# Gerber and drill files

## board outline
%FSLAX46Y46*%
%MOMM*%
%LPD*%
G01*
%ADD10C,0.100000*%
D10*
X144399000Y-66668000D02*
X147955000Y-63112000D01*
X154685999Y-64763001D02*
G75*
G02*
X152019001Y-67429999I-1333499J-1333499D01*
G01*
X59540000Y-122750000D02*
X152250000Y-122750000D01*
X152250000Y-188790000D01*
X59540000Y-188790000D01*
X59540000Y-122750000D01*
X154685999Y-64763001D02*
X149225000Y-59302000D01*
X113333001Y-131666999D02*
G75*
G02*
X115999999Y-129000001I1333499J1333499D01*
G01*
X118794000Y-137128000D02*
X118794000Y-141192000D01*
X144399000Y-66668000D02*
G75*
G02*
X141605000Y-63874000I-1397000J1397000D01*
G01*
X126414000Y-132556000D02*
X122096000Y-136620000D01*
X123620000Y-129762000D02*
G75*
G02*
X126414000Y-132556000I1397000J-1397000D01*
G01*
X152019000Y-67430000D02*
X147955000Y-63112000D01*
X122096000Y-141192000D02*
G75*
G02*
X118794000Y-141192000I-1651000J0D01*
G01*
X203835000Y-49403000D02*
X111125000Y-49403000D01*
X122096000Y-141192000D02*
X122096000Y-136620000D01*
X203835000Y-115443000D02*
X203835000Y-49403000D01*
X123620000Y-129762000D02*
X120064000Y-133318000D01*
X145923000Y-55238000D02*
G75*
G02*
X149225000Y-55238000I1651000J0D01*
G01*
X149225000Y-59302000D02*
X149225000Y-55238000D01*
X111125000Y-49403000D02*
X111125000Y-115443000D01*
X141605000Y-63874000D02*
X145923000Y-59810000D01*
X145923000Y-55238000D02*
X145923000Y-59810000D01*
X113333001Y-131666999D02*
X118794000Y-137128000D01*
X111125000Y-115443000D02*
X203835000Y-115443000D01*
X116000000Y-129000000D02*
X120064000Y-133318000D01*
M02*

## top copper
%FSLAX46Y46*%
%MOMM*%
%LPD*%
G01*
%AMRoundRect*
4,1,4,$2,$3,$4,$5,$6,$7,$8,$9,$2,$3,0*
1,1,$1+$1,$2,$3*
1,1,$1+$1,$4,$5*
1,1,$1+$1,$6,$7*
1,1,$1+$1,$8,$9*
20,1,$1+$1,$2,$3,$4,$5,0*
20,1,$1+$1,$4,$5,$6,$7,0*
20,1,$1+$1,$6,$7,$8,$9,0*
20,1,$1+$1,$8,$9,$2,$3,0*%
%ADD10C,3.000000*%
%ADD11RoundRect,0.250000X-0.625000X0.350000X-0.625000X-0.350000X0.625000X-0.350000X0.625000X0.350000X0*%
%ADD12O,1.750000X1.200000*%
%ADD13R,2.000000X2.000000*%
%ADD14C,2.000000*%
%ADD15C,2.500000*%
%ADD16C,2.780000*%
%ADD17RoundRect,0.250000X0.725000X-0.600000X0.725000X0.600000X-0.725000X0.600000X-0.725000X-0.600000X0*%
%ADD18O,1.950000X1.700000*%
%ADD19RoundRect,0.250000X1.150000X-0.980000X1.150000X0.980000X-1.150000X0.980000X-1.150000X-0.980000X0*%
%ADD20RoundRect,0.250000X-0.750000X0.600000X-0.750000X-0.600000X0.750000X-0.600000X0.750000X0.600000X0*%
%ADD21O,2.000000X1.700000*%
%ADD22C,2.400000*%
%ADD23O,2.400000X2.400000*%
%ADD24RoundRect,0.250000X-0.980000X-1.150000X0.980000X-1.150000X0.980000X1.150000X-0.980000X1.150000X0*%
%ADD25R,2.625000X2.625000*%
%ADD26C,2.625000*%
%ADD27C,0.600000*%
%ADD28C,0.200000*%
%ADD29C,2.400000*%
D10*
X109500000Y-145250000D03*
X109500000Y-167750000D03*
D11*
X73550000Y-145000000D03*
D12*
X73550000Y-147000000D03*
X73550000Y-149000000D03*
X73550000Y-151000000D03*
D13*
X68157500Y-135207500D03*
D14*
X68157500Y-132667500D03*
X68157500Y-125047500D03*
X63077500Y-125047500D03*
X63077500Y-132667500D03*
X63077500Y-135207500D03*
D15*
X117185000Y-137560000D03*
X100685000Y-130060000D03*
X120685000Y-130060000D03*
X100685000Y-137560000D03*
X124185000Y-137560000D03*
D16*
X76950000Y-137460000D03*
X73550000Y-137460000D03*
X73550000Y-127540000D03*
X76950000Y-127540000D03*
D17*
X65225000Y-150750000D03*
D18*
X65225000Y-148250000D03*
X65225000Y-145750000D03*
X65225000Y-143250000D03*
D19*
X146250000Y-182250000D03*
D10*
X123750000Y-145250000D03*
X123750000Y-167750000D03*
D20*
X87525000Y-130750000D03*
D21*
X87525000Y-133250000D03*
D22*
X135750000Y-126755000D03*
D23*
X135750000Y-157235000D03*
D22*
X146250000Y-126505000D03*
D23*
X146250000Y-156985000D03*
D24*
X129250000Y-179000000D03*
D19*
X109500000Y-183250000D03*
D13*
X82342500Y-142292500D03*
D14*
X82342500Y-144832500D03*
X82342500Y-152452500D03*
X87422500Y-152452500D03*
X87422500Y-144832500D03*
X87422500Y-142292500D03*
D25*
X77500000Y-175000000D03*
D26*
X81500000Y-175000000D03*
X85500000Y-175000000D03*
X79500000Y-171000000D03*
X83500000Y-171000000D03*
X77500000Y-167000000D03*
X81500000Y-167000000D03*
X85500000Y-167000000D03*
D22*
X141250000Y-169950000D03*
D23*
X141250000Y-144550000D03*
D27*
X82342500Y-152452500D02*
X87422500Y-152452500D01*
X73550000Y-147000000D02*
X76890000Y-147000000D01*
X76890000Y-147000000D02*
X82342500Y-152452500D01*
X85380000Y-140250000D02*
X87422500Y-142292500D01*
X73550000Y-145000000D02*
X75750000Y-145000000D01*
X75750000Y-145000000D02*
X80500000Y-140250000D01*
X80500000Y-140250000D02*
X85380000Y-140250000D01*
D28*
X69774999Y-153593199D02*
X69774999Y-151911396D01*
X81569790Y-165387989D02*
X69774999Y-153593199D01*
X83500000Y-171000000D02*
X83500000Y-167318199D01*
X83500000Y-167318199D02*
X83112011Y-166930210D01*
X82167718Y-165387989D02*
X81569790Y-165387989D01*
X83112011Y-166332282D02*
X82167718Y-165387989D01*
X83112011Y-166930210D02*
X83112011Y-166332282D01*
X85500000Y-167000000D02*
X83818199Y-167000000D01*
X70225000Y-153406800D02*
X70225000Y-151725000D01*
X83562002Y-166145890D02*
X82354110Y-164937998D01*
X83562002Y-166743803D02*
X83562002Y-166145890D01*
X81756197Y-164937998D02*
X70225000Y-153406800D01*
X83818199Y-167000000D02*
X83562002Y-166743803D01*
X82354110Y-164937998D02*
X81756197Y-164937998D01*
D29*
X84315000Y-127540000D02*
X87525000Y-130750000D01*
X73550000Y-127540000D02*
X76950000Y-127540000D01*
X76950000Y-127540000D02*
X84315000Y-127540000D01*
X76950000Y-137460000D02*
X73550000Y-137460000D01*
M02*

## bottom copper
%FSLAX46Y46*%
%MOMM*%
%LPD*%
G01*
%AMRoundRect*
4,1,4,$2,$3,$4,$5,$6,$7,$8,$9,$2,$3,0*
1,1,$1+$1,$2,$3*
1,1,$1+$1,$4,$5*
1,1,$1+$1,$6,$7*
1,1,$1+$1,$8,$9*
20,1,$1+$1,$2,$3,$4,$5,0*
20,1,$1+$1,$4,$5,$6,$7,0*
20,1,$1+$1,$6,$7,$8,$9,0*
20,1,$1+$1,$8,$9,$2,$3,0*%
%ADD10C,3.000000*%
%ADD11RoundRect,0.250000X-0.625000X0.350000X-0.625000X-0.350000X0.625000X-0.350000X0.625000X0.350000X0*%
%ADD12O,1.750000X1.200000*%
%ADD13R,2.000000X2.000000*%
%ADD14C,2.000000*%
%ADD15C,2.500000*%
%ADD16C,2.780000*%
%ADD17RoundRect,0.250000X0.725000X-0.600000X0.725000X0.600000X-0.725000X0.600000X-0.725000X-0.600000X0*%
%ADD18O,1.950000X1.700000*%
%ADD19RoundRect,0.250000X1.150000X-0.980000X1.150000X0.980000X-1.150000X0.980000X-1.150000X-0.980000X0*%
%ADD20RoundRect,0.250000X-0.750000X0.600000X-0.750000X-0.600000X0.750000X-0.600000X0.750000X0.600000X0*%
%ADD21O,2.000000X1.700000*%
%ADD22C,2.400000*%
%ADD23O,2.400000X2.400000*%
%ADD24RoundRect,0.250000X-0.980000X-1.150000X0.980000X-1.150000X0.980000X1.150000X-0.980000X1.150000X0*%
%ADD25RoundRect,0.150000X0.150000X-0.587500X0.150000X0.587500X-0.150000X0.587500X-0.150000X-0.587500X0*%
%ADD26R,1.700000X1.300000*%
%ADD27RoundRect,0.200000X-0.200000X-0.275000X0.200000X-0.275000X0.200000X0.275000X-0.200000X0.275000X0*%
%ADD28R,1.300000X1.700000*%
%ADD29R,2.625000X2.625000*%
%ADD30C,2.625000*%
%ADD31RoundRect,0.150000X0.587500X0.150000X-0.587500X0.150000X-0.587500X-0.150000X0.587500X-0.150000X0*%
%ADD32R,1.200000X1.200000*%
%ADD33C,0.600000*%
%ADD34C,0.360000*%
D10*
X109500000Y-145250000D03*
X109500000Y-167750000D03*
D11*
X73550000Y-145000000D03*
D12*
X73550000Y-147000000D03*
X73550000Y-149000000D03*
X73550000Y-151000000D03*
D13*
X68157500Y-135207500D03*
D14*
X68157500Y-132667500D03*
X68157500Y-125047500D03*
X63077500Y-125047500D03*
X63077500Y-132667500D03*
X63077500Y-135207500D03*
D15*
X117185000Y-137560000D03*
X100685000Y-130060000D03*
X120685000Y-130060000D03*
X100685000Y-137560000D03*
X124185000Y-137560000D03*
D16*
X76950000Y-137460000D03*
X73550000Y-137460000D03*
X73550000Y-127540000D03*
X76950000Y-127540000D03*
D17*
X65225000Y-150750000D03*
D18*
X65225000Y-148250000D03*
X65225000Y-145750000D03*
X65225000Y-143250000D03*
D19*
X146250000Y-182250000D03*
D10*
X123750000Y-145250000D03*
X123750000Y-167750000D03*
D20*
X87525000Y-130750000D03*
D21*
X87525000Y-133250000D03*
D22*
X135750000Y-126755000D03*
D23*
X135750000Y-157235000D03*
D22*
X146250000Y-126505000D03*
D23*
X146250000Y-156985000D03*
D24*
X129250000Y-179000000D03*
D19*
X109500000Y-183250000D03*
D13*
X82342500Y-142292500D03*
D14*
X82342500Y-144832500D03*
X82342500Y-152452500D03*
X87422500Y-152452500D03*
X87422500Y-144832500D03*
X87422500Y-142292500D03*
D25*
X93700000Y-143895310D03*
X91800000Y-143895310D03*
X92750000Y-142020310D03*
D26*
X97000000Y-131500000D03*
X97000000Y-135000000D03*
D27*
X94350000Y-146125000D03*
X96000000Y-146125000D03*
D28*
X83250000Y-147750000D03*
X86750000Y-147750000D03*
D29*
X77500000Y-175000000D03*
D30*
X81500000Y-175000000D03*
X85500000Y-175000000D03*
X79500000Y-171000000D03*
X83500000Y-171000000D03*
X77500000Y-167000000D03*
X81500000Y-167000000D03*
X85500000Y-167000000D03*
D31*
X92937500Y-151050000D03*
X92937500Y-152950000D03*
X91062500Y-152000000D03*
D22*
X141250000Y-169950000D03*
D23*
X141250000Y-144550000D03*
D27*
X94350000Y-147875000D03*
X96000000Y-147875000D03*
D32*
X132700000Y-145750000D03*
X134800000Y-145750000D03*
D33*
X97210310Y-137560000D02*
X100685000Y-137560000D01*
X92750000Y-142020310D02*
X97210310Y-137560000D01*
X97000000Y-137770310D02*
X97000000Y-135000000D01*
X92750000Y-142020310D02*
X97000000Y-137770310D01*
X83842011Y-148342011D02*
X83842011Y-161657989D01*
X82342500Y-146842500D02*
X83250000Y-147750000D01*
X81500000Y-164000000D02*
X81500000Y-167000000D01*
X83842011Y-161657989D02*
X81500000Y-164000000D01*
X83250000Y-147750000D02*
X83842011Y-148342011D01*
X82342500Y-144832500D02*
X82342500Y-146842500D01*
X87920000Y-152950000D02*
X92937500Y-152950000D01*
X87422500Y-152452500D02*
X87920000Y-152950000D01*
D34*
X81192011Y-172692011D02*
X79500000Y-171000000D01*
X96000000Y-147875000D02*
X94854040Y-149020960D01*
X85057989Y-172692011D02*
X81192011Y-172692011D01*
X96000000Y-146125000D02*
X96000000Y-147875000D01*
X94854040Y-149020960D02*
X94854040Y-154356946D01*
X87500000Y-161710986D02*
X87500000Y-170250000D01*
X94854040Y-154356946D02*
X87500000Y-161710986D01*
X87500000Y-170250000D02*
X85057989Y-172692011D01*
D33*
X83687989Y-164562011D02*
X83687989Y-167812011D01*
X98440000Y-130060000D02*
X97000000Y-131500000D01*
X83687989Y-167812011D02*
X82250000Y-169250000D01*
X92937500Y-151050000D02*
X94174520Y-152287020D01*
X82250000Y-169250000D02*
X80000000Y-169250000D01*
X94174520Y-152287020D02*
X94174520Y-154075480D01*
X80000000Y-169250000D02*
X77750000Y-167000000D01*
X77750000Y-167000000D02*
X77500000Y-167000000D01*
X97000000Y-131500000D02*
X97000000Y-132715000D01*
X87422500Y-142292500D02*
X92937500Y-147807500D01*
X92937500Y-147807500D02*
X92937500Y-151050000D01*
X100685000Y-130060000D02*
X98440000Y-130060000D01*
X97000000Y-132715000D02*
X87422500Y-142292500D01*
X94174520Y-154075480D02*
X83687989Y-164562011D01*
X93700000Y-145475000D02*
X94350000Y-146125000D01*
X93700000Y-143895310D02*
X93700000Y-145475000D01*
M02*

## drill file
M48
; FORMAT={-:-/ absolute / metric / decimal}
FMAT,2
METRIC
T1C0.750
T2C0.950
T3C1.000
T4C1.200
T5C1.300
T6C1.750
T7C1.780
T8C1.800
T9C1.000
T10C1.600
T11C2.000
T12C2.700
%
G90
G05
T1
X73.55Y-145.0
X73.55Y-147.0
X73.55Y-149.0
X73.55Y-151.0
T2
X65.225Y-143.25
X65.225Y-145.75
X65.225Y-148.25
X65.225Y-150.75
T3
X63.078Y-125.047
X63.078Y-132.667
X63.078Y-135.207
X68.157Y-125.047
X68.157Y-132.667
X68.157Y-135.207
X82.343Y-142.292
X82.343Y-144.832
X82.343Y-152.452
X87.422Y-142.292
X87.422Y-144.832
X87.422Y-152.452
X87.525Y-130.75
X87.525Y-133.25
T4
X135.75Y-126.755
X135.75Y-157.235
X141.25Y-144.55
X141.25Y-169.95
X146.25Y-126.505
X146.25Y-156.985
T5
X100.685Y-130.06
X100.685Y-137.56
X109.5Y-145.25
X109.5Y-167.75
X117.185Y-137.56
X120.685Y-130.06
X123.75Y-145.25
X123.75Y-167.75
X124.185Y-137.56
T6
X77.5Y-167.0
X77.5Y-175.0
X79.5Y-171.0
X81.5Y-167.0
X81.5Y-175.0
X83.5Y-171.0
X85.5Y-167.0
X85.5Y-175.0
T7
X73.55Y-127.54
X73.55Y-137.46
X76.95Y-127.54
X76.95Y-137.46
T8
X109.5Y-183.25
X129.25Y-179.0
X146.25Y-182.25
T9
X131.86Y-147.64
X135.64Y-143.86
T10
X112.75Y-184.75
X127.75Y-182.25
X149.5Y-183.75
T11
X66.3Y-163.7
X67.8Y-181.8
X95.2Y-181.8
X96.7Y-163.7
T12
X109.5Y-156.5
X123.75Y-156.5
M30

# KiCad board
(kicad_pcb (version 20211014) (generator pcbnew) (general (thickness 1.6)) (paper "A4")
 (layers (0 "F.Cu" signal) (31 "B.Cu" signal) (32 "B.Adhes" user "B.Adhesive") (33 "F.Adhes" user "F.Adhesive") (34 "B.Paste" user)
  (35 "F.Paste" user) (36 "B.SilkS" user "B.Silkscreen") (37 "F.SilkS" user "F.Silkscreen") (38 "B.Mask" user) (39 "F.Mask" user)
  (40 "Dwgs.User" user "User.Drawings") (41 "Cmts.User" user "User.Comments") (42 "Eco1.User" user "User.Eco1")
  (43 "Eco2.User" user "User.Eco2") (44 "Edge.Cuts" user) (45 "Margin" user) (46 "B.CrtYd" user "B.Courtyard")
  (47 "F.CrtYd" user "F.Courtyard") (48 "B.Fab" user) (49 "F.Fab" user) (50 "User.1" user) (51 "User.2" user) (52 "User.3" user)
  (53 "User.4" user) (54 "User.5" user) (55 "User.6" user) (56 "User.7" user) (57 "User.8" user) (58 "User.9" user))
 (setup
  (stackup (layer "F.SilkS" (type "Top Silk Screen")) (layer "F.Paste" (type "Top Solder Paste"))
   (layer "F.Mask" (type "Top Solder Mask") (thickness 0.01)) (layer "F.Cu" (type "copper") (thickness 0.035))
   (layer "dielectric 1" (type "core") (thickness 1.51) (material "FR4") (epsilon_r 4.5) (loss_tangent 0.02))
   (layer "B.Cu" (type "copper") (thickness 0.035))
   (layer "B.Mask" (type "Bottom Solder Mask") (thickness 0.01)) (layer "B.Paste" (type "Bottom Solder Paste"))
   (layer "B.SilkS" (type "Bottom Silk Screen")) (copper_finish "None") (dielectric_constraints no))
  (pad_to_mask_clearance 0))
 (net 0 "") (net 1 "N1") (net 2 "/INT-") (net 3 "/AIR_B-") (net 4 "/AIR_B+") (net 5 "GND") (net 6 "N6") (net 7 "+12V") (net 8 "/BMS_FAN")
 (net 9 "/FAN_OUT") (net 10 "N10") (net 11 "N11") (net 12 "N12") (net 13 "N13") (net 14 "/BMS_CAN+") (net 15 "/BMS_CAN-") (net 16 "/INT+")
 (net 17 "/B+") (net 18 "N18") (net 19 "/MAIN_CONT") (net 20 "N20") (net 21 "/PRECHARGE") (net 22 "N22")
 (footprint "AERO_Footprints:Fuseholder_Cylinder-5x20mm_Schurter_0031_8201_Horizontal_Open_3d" (layer "F.Cu") (at 109.5 145.25 -90)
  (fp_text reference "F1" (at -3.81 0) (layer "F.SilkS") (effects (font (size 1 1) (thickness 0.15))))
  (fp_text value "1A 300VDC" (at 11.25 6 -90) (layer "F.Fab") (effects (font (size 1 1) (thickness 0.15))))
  (pad "" np_thru_hole circle locked (at 11.25 0 270) (size 2.7 2.7) (drill 2.7) (layers *.Cu *.Mask))
  (pad "1" thru_hole circle locked (at 0 0 270) (size 3 3) (drill 1.3) (layers *.Cu *.Mask) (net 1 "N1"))
  (pad "2" thru_hole circle locked (at 22.5 0 270) (size 3 3) (drill 1.3) (layers *.Cu *.Mask) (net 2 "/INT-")))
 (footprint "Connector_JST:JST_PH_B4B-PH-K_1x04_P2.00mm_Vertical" (layer "F.Cu") (at 73.55 145 -90)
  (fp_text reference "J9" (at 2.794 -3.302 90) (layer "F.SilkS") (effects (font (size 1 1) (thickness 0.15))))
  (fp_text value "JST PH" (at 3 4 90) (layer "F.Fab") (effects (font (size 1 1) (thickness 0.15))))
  (pad "1" thru_hole roundrect locked (at 0 0 270) (size 1.2 1.75) (drill 0.75) (layers *.Cu *.Mask) (roundrect_rratio 0.208333)
   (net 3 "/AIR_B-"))
  (pad "2" thru_hole oval locked (at 2 0 270) (size 1.2 1.75) (drill 0.75) (layers *.Cu *.Mask) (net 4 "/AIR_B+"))
  (pad "3" thru_hole oval locked (at 4 0 270) (size 1.2 1.75) (drill 0.75) (layers *.Cu *.Mask) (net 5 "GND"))
  (pad "4" thru_hole oval locked (at 6 0 270) (size 1.2 1.75) (drill 0.75) (layers *.Cu *.Mask) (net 5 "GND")))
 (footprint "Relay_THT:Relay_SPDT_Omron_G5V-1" (layer "F.Cu") (at 68.1575 135.2075 180)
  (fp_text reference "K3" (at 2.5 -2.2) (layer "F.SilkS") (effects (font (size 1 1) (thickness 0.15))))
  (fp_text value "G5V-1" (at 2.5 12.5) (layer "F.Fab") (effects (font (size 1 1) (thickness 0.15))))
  (pad "1" thru_hole rect locked (at 0 0 180) (size 2 2) (drill 1) (layers *.Cu *.Mask) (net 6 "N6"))
  (pad "2" thru_hole circle locked (at 0 2.54 180) (size 2 2) (drill 1) (layers *.Cu *.Mask) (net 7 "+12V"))
  (pad "5" thru_hole circle locked (at 0 10.16 180) (size 2 2) (drill 1) (layers *.Cu *.Mask) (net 7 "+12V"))
  (pad "6" thru_hole circle locked (at 5.08 10.16 180) (size 2 2) (drill 1) (layers *.Cu *.Mask) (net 7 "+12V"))
  (pad "9" thru_hole circle locked (at 5.08 2.54 180) (size 2 2) (drill 1) (layers *.Cu *.Mask) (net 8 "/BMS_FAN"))
  (pad "10" thru_hole circle locked (at 5.08 0 180) (size 2 2) (drill 1) (layers *.Cu *.Mask) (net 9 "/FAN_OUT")))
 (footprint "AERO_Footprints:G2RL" (layer "F.Cu") (at 113.385 133.75)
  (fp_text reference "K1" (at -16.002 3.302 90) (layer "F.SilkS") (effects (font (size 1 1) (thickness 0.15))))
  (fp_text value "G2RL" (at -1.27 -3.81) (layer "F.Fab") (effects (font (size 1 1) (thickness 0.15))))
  (pad "1" thru_hole circle locked (at 3.8 3.81) (size 2.5 2.5) (drill 1.3) (layers *.Cu *.Mask) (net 1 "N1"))
  (pad "2" thru_hole circle locked (at -12.7 -3.69) (size 2.5 2.5) (drill 1.3) (layers *.Cu *.Mask) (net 3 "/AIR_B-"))
  (pad "5" thru_hole circle locked (at 7.3 -3.69) (size 2.5 2.5) (drill 1.3) (layers *.Cu *.Mask) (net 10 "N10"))
  (pad "9" thru_hole circle locked (at -12.7 3.81) (size 2.5 2.5) (drill 1.3) (layers *.Cu *.Mask) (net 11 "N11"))
  (pad "10" thru_hole circle locked (at 10.8 3.81) (size 2.5 2.5) (drill 1.3) (layers *.Cu *.Mask) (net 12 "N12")))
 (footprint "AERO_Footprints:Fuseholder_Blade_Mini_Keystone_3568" (layer "F.Cu") (at 73.55 137.46 90)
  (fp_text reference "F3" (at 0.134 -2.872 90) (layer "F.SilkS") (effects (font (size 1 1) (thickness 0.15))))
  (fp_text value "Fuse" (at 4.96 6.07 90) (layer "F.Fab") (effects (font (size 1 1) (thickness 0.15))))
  (pad "1" thru_hole circle locked (at 0 3.4 90) (size 2.78 2.78) (drill 1.78) (layers *.Cu *.Mask) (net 9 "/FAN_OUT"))
  (pad "1" thru_hole circle locked (at 0 0 90) (size 2.78 2.78) (drill 1.78) (layers *.Cu *.Mask) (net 9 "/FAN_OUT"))
  (pad "2" thru_hole circle locked (at 9.92 0 90) (size 2.78 2.78) (drill 1.78) (layers *.Cu *.Mask) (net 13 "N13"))
  (pad "2" thru_hole circle locked (at 9.92 3.4 90) (size 2.78 2.78) (drill 1.78) (layers *.Cu *.Mask) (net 13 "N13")))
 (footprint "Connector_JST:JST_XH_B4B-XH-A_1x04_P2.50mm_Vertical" (layer "F.Cu") (at 65.225 150.75 90)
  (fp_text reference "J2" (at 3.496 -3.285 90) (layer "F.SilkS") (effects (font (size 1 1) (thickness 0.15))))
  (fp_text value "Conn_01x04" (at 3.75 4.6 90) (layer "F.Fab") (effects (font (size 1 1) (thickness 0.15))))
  (pad "1" thru_hole roundrect locked (at 0 0 90) (size 1.7 1.95) (drill 0.95) (layers *.Cu *.Mask) (roundrect_rratio 0.147059)
   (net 7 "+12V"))
  (pad "2" thru_hole oval locked (at 2.5 0 90) (size 1.7 1.95) (drill 0.95) (layers *.Cu *.Mask) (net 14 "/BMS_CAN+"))
  (pad "3" thru_hole oval locked (at 5 0 90) (size 1.7 1.95) (drill 0.95) (layers *.Cu *.Mask) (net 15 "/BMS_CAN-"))
  (pad "4" thru_hole oval locked (at 7.5 0 90) (size 1.7 1.95) (drill 0.95) (layers *.Cu *.Mask) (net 5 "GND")))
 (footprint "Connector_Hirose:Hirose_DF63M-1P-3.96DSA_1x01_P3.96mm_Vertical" (layer "F.Cu") (at 146.25 182.25 90)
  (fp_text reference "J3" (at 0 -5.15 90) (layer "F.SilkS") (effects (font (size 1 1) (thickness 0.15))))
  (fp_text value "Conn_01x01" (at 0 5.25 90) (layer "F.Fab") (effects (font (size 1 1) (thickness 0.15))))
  (pad "" np_thru_hole circle locked (at -1.5 3.25 90) (size 1.6 1.6) (drill 1.6) (layers *.Cu *.Mask))
  (pad "1" thru_hole roundrect locked (at 0 0 90) (size 2.46 2.8) (drill 1.8) (layers *.Cu *.Mask) (roundrect_rratio 0.101626)
   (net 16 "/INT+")))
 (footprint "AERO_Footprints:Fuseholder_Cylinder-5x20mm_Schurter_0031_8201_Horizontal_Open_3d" (layer "F.Cu") (at 123.75 145.25 -90)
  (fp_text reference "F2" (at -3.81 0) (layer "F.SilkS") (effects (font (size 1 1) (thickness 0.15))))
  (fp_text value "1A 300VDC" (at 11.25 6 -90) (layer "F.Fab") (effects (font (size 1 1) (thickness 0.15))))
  (pad "" np_thru_hole circle locked (at 11.25 0 270) (size 2.7 2.7) (drill 2.7) (layers *.Cu *.Mask))
  (pad "1" thru_hole circle locked (at 0 0 270) (size 3 3) (drill 1.3) (layers *.Cu *.Mask) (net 12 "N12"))
  (pad "2" thru_hole circle locked (at 22.5 0 270) (size 3 3) (drill 1.3) (layers *.Cu *.Mask) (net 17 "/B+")))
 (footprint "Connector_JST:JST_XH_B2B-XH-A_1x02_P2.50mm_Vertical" (layer "F.Cu") (at 87.525 130.75 -90)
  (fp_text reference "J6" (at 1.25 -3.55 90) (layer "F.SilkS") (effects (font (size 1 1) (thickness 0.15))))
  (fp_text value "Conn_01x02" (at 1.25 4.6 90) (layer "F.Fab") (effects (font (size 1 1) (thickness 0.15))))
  (pad "1" thru_hole roundrect locked (at 0 0 270) (size 1.7 2) (drill 1) (layers *.Cu *.Mask) (roundrect_rratio 0.147059) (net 13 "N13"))
  (pad "2" thru_hole oval locked (at 2.5 0 270) (size 1.7 2) (drill 1) (layers *.Cu *.Mask) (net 5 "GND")))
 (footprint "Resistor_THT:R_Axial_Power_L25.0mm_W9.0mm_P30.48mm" (layer "F.Cu") (at 135.75 126.755 -90)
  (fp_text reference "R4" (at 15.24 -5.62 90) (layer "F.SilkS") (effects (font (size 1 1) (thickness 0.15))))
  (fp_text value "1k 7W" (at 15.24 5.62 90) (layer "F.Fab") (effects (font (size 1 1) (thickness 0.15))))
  (pad "1" thru_hole circle locked (at 0 0 270) (size 2.4 2.4) (drill 1.2) (layers *.Cu *.Mask) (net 10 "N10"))
  (pad "2" thru_hole oval locked (at 30.48 0 270) (size 2.4 2.4) (drill 1.2) (layers *.Cu *.Mask) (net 16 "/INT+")))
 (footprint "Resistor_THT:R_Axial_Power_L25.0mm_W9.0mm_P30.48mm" (layer "F.Cu") (at 146.25 126.505 -90)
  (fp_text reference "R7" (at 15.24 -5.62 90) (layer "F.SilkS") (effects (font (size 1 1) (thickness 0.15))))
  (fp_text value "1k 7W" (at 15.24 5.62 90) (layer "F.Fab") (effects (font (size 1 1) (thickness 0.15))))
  (pad "1" thru_hole circle locked (at 0 0 270) (size 2.4 2.4) (drill 1.2) (layers *.Cu *.Mask) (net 10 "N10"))
  (pad "2" thru_hole oval locked (at 30.48 0 270) (size 2.4 2.4) (drill 1.2) (layers *.Cu *.Mask) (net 16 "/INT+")))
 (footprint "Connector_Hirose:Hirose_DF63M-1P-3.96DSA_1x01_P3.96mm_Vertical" (layer "F.Cu") (at 129.25 179)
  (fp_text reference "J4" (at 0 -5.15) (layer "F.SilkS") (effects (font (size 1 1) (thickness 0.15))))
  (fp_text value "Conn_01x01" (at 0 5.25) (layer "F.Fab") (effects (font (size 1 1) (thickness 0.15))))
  (pad "" np_thru_hole circle locked (at -1.5 3.25) (size 1.6 1.6) (drill 1.6) (layers *.Cu *.Mask))
  (pad "1" thru_hole roundrect locked (at 0 0) (size 2.46 2.8) (drill 1.8) (layers *.Cu *.Mask) (roundrect_rratio 0.101626) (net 17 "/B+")))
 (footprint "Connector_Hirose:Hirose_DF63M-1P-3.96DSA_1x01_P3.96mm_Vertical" (layer "F.Cu") (at 109.5 183.25 90)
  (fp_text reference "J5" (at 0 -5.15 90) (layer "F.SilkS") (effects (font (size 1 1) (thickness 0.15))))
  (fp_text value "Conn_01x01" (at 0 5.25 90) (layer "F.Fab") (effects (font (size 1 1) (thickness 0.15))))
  (pad "" np_thru_hole circle locked (at -1.5 3.25 90) (size 1.6 1.6) (drill 1.6) (layers *.Cu *.Mask))
  (pad "1" thru_hole roundrect locked (at 0 0 90) (size 2.46 2.8) (drill 1.8) (layers *.Cu *.Mask) (roundrect_rratio 0.101626)
   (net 2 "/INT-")))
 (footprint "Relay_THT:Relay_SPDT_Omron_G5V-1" (layer "F.Cu") (at 82.3425 142.2925)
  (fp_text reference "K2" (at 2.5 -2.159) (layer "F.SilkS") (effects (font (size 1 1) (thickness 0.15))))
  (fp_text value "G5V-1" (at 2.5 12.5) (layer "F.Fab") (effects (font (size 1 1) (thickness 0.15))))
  (pad "1" thru_hole rect locked (at 0 0) (size 2 2) (drill 1) (layers *.Cu *.Mask) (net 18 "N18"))
  (pad "2" thru_hole circle locked (at 0 2.54) (size 2 2) (drill 1) (layers *.Cu *.Mask) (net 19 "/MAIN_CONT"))
  (pad "5" thru_hole circle locked (at 0 10.16) (size 2 2) (drill 1) (layers *.Cu *.Mask) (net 4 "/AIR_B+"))
  (pad "6" thru_hole circle locked (at 5.08 10.16) (size 2 2) (drill 1) (layers *.Cu *.Mask) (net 4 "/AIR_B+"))
  (pad "9" thru_hole circle locked (at 5.08 2.54) (size 2 2) (drill 1) (layers *.Cu *.Mask) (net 5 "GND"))
  (pad "10" thru_hole circle locked (at 5.08 0) (size 2 2) (drill 1) (layers *.Cu *.Mask) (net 3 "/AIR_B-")))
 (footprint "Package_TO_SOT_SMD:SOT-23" (layer "B.Cu") (at 92.75 142.95781 90)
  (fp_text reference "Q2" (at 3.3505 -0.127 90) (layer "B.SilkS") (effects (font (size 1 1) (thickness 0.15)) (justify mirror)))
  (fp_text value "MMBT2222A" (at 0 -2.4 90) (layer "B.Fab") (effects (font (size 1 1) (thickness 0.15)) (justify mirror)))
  (pad "1" smd roundrect locked (at -0.9375 0.95 90) (size 1.475 0.6) (layers "B.Cu" "B.Paste" "B.Mask") (roundrect_rratio 0.25)
   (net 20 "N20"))
  (pad "2" smd roundrect locked (at -0.9375 -0.95 90) (size 1.475 0.6) (layers "B.Cu" "B.Paste" "B.Mask") (roundrect_rratio 0.25)
   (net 5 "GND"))
  (pad "3" smd roundrect locked (at 0.9375 0 90) (size 1.475 0.6) (layers "B.Cu" "B.Paste" "B.Mask") (roundrect_rratio 0.25) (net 11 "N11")))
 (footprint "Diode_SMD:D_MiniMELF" (layer "B.Cu") (at 97 133.25 -90)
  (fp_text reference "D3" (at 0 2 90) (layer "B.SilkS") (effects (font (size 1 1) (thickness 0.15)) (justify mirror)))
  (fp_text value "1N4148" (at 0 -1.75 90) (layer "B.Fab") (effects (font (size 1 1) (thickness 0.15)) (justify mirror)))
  (pad "1" smd rect locked (at -1.75 0 270) (size 1.3 1.7) (layers "B.Cu" "B.Paste" "B.Mask") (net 3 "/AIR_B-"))
  (pad "2" smd rect locked (at 1.75 0 270) (size 1.3 1.7) (layers "B.Cu" "B.Paste" "B.Mask") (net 11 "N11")))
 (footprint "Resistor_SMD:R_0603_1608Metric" (layer "B.Cu") (at 95.175 146.125)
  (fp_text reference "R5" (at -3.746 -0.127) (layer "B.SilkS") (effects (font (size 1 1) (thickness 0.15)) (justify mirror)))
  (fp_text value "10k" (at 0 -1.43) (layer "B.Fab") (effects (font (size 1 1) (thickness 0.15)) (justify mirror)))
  (pad "1" smd roundrect locked (at -0.825 0) (size 0.8 0.95) (layers "B.Cu" "B.Paste" "B.Mask") (roundrect_rratio 0.25) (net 20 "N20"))
  (pad "2" smd roundrect locked (at 0.825 0) (size 0.8 0.95) (layers "B.Cu" "B.Paste" "B.Mask") (roundrect_rratio 0.25)
   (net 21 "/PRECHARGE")))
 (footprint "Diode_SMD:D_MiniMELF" (layer "B.Cu") (at 85 147.75)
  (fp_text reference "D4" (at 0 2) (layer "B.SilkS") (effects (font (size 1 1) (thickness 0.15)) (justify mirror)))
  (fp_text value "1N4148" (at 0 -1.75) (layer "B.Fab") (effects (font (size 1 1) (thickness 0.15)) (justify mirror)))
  (pad "1" smd rect locked (at -1.75 0) (size 1.3 1.7) (layers "B.Cu" "B.Paste" "B.Mask") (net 19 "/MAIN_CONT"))
  (pad "2" smd rect locked (at 1.75 0) (size 1.3 1.7) (layers "B.Cu" "B.Paste" "B.Mask") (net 5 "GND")))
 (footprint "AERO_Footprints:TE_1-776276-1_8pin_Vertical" (layer "B.Cu") (at 81.5 171)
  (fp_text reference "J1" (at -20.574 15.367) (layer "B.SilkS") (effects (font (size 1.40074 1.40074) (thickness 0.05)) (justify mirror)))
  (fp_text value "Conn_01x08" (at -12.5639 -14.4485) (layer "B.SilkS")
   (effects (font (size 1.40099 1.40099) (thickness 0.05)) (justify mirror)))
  (pad "" np_thru_hole circle locked (at 13.7 10.8) (size 2 2) (drill 2) (layers *.Cu *.Mask "B.SilkS"))
  (pad "" np_thru_hole circle locked (at -15.2 -7.3) (size 2 2) (drill 2) (layers *.Cu *.Mask "B.SilkS"))
  (pad "" np_thru_hole circle locked (at 15.2 -7.3) (size 2 2) (drill 2) (layers *.Cu *.Mask "B.SilkS"))
  (pad "" np_thru_hole circle locked (at -13.7 10.8) (size 2 2) (drill 2) (layers *.Cu *.Mask "B.SilkS"))
  (pad "1" thru_hole rect locked (at -4 4) (size 2.625 2.625) (drill 1.75) (layers *.Cu *.Mask) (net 5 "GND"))
  (pad "2" thru_hole circle locked (at 0 4) (size 2.625 2.625) (drill 1.75) (layers *.Cu *.Mask) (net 8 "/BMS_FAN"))
  (pad "3" thru_hole circle locked (at 4 4) (size 2.625 2.625) (drill 1.75) (layers *.Cu *.Mask) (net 7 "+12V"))
  (pad "4" thru_hole circle locked (at -2 0) (size 2.625 2.625) (drill 1.75) (layers *.Cu *.Mask) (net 21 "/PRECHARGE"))
  (pad "5" thru_hole circle locked (at 2 0) (size 2.625 2.625) (drill 1.75) (layers *.Cu *.Mask) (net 14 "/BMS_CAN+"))
  (pad "6" thru_hole circle locked (at -4 -4) (size 2.625 2.625) (drill 1.75) (layers *.Cu *.Mask) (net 3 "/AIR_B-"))
  (pad "7" thru_hole circle locked (at 0 -4) (size 2.625 2.625) (drill 1.75) (layers *.Cu *.Mask) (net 19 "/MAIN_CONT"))
  (pad "8" thru_hole circle locked (at 4 -4) (size 2.625 2.625) (drill 1.75) (layers *.Cu *.Mask) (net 15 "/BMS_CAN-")))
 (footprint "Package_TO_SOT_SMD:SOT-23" (layer "B.Cu") (at 92 152 180)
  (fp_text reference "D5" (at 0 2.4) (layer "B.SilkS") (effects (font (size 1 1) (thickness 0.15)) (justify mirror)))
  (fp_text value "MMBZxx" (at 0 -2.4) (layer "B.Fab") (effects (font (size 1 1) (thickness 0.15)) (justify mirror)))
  (pad "1" smd roundrect locked (at -0.9375 0.95 180) (size 1.475 0.6) (layers "B.Cu" "B.Paste" "B.Mask") (roundrect_rratio 0.25)
   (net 3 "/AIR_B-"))
  (pad "2" smd roundrect locked (at -0.9375 -0.95 180) (size 1.475 0.6) (layers "B.Cu" "B.Paste" "B.Mask") (roundrect_rratio 0.25)
   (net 4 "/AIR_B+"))
  (pad "3" smd roundrect locked (at 0.9375 0 180) (size 1.475 0.6) (layers "B.Cu" "B.Paste" "B.Mask") (roundrect_rratio 0.25) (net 5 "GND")))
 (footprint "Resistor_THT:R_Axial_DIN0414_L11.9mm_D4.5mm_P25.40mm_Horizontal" (layer "B.Cu") (at 141.25 169.95 90)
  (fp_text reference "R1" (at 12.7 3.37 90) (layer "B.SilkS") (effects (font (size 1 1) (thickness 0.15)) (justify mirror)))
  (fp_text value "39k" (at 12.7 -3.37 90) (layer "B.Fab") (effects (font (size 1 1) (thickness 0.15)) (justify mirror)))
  (pad "1" thru_hole circle locked (at 0 0 90) (size 2.4 2.4) (drill 1.2) (layers *.Cu *.Mask) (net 16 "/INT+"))
  (pad "2" thru_hole oval locked (at 25.4 0 90) (size 2.4 2.4) (drill 1.2) (layers *.Cu *.Mask) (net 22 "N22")))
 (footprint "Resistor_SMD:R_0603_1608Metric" (layer "B.Cu") (at 95.175 147.875)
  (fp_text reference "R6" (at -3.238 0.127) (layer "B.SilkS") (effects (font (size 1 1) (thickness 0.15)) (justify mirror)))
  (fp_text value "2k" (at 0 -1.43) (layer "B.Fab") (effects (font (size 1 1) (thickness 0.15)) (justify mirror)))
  (pad "1" smd roundrect locked (at -0.825 0) (size 0.8 0.95) (layers "B.Cu" "B.Paste" "B.Mask") (roundrect_rratio 0.25) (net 5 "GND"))
  (pad "2" smd roundrect locked (at 0.825 0) (size 0.8 0.95) (layers "B.Cu" "B.Paste" "B.Mask") (roundrect_rratio 0.25)
   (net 21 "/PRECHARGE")))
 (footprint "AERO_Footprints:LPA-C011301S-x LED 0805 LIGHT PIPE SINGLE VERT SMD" (layer "B.Cu") (at 133.75 145.75)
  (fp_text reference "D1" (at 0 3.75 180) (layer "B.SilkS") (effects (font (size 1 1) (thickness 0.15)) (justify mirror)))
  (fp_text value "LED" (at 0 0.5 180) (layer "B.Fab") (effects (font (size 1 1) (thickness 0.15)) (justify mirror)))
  (pad "" np_thru_hole circle locked (at 1.89 -1.89) (size 1 1) (drill 1) (layers *.Cu *.Mask))
  (pad "" np_thru_hole circle locked (at -1.89 1.89) (size 1 1) (drill 1) (layers *.Cu *.Mask))
  (pad "1" smd rect locked (at -1.05 0) (size 1.2 1.2) (layers "B.Cu" "B.Paste" "B.Mask") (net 2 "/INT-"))
  (pad "2" smd rect locked (at 1.05 0) (size 1.2 1.2) (layers "B.Cu" "B.Paste" "B.Mask") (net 22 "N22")))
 (gr_line (start 144.399 66.668) (end 147.955 63.112) (layer "Edge.Cuts") (width 0.1))
 (gr_arc (start 154.685999 64.763001) (mid 154.685999 67.429999) (end 152.019001 67.429999) (layer "Edge.Cuts") (width 0.1))
 (gr_rect (start 59.54 188.79) (end 152.25 122.75) (layer "Edge.Cuts") (width 0.1) (fill none))
 (gr_line (start 154.685999 64.763001) (end 149.225 59.302) (layer "Edge.Cuts") (width 0.1))
 (gr_arc (start 113.333001 131.666999) (mid 113.333001 129.000001) (end 115.999999 129.000001) (layer "Edge.Cuts") (width 0.1))
 (gr_line (start 118.794 137.128) (end 118.794 141.192) (layer "Edge.Cuts") (width 0.1))
 (gr_arc (start 144.399 66.668) (mid 141.605 66.668) (end 141.605 63.874) (layer "Edge.Cuts") (width 0.1))
 (gr_line (start 126.414 132.556) (end 122.096 136.62) (layer "Edge.Cuts") (width 0.1))
 (gr_arc (start 123.62 129.762) (mid 126.414 129.762) (end 126.414 132.556) (layer "Edge.Cuts") (width 0.1))
 (gr_line (start 152.019 67.43) (end 147.955 63.112) (layer "Edge.Cuts") (width 0.1))
 (gr_arc (start 122.096 141.192) (mid 120.445 142.843) (end 118.794 141.192) (layer "Edge.Cuts") (width 0.1))
 (gr_line (start 203.835 49.403) (end 111.125 49.403) (layer "Edge.Cuts") (width 0.1))
 (gr_line (start 122.096 141.192) (end 122.096 136.62) (layer "Edge.Cuts") (width 0.1))
 (gr_line (start 203.835 115.443) (end 203.835 49.403) (layer "Edge.Cuts") (width 0.1))
 (gr_line (start 123.62 129.762) (end 120.064 133.318) (layer "Edge.Cuts") (width 0.1))
 (gr_arc (start 145.923 55.238) (mid 147.574 53.587) (end 149.225 55.238) (layer "Edge.Cuts") (width 0.1))
 (gr_line (start 149.225 59.302) (end 149.225 55.238) (layer "Edge.Cuts") (width 0.1))
 (gr_line (start 111.125 49.403) (end 111.125 115.443) (layer "Edge.Cuts") (width 0.1))
 (gr_line (start 141.605 63.874) (end 145.923 59.81) (layer "Edge.Cuts") (width 0.1))
 (gr_line (start 145.923 55.238) (end 145.923 59.81) (layer "Edge.Cuts") (width 0.1))
 (gr_line (start 113.333001 131.666999) (end 118.794 137.128) (layer "Edge.Cuts") (width 0.1))
 (gr_line (start 111.125 115.443) (end 203.835 115.443) (layer "Edge.Cuts") (width 0.1))
 (gr_line (start 116 129) (end 120.064 133.318) (layer "Edge.Cuts") (width 0.1))
 (segment (start 97.21031 137.56) (end 100.685 137.56) (width 0.6) (layer "B.Cu") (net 11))
 (segment (start 92.75 142.02031) (end 97.21031 137.56) (width 0.6) (layer "B.Cu") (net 11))
 (segment (start 97 137.77031) (end 97 135) (width 0.6) (layer "B.Cu") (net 11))
 (segment (start 92.75 142.02031) (end 97 137.77031) (width 0.6) (layer "B.Cu") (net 11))
 (segment (start 83.842011 148.342011) (end 83.842011 161.657989) (width 0.6) (layer "B.Cu") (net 19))
 (segment (start 82.3425 146.8425) (end 83.25 147.75) (width 0.6) (layer "B.Cu") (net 19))
 (segment (start 81.5 164) (end 81.5 167) (width 0.6) (layer "B.Cu") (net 19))
 (segment (start 83.842011 161.657989) (end 81.5 164) (width 0.6) (layer "B.Cu") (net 19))
 (segment (start 83.25 147.75) (end 83.842011 148.342011) (width 0.6) (layer "B.Cu") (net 19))
 (segment (start 82.3425 144.8325) (end 82.3425 146.8425) (width 0.6) (layer "B.Cu") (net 19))
 (segment (start 82.3425 152.4525) (end 87.4225 152.4525) (width 0.6) (layer "F.Cu") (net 4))
 (segment (start 73.55 147) (end 76.89 147) (width 0.6) (layer "F.Cu") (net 4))
 (segment (start 76.89 147) (end 82.3425 152.4525) (width 0.6) (layer "F.Cu") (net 4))
 (segment (start 87.92 152.95) (end 92.9375 152.95) (width 0.6) (layer "B.Cu") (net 4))
 (segment (start 87.4225 152.4525) (end 87.92 152.95) (width 0.6) (layer "B.Cu") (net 4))
 (segment (start 81.192011 172.692011) (end 79.5 171) (width 0.36) (layer "B.Cu") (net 21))
 (segment (start 96 147.875) (end 94.85404 149.02096) (width 0.36) (layer "B.Cu") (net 21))
 (segment (start 85.057989 172.692011) (end 81.192011 172.692011) (width 0.36) (layer "B.Cu") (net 21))
 (segment (start 96 146.125) (end 96 147.875) (width 0.36) (layer "B.Cu") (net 21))
 (segment (start 94.85404 149.02096) (end 94.85404 154.356946) (width 0.36) (layer "B.Cu") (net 21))
 (segment (start 87.5 161.710986) (end 87.5 170.25) (width 0.36) (layer "B.Cu") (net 21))
 (segment (start 94.85404 154.356946) (end 87.5 161.710986) (width 0.36) (layer "B.Cu") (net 21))
 (segment (start 87.5 170.25) (end 85.057989 172.692011) (width 0.36) (layer "B.Cu") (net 21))
 (segment (start 85.38 140.25) (end 87.4225 142.2925) (width 0.6) (layer "F.Cu") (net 3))
 (segment (start 73.55 145) (end 75.75 145) (width 0.6) (layer "F.Cu") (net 3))
 (segment (start 75.75 145) (end 80.5 140.25) (width 0.6) (layer "F.Cu") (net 3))
 (segment (start 80.5 140.25) (end 85.38 140.25) (width 0.6) (layer "F.Cu") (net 3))
 (segment (start 83.687989 164.562011) (end 83.687989 167.812011) (width 0.6) (layer "B.Cu") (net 3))
 (segment (start 98.44 130.06) (end 97 131.5) (width 0.6) (layer "B.Cu") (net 3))
 (segment (start 83.687989 167.812011) (end 82.25 169.25) (width 0.6) (layer "B.Cu") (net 3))
 (segment (start 92.9375 151.05) (end 94.17452 152.28702) (width 0.6) (layer "B.Cu") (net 3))
 (segment (start 82.25 169.25) (end 80 169.25) (width 0.6) (layer "B.Cu") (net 3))
 (segment (start 94.17452 152.28702) (end 94.17452 154.07548) (width 0.6) (layer "B.Cu") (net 3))
 (segment (start 80 169.25) (end 77.75 167) (width 0.6) (layer "B.Cu") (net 3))
 (segment (start 77.75 167) (end 77.5 167) (width 0.6) (layer "B.Cu") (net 3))
 (segment (start 97 131.5) (end 97 132.715) (width 0.6) (layer "B.Cu") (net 3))
 (segment (start 87.4225 142.2925) (end 92.9375 147.8075) (width 0.6) (layer "B.Cu") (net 3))
 (segment (start 92.9375 147.8075) (end 92.9375 151.05) (width 0.6) (layer "B.Cu") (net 3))
 (segment (start 100.685 130.06) (end 98.44 130.06) (width 0.6) (layer "B.Cu") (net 3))
 (segment (start 97 132.715) (end 87.4225 142.2925) (width 0.6) (layer "B.Cu") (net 3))
 (segment (start 94.17452 154.07548) (end 83.687989 164.562011) (width 0.6) (layer "B.Cu") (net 3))
 (segment (start 69.774999 153.593199) (end 69.774999 151.911396) (width 0.2) (layer "F.Cu") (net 14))
 (segment (start 81.56979 165.387989) (end 69.774999 153.593199) (width 0.2) (layer "F.Cu") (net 14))
 (segment (start 83.5 171) (end 83.5 167.318199) (width 0.2) (layer "F.Cu") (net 14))
 (segment (start 83.5 167.318199) (end 83.112011 166.93021) (width 0.2) (layer "F.Cu") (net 14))
 (segment (start 82.167718 165.387989) (end 81.56979 165.387989) (width 0.2) (layer "F.Cu") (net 14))
 (segment (start 83.112011 166.332282) (end 82.167718 165.387989) (width 0.2) (layer "F.Cu") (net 14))
 (segment (start 83.112011 166.93021) (end 83.112011 166.332282) (width 0.2) (layer "F.Cu") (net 14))
 (segment (start 85.5 167) (end 83.818199 167) (width 0.2) (layer "F.Cu") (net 15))
 (segment (start 70.225 153.4068) (end 70.225 151.725) (width 0.2) (layer "F.Cu") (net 15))
 (segment (start 83.562002 166.14589) (end 82.35411 164.937998) (width 0.2) (layer "F.Cu") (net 15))
 (segment (start 83.562002 166.743803) (end 83.562002 166.14589) (width 0.2) (layer "F.Cu") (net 15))
 (segment (start 81.756197 164.937998) (end 70.225 153.4068) (width 0.2) (layer "F.Cu") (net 15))
 (segment (start 83.818199 167) (end 83.562002 166.743803) (width 0.2) (layer "F.Cu") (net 15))
 (segment (start 82.35411 164.937998) (end 81.756197 164.937998) (width 0.2) (layer "F.Cu") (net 15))
 (segment (start 93.7 145.475) (end 94.35 146.125) (width 0.6) (layer "B.Cu") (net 20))
 (segment (start 93.7 143.89531) (end 93.7 145.475) (width 0.6) (layer "B.Cu") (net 20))
 (segment (start 84.315 127.54) (end 87.525 130.75) (width 2.4) (layer "F.Cu") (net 13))
 (segment (start 73.55 127.54) (end 76.95 127.54) (width 2.4) (layer "F.Cu") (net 13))
 (segment (start 76.95 127.54) (end 84.315 127.54) (width 2.4) (layer "F.Cu") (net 13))
 (segment (start 76.95 137.46) (end 73.55 137.46) (width 2.4) (layer "F.Cu") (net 9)))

